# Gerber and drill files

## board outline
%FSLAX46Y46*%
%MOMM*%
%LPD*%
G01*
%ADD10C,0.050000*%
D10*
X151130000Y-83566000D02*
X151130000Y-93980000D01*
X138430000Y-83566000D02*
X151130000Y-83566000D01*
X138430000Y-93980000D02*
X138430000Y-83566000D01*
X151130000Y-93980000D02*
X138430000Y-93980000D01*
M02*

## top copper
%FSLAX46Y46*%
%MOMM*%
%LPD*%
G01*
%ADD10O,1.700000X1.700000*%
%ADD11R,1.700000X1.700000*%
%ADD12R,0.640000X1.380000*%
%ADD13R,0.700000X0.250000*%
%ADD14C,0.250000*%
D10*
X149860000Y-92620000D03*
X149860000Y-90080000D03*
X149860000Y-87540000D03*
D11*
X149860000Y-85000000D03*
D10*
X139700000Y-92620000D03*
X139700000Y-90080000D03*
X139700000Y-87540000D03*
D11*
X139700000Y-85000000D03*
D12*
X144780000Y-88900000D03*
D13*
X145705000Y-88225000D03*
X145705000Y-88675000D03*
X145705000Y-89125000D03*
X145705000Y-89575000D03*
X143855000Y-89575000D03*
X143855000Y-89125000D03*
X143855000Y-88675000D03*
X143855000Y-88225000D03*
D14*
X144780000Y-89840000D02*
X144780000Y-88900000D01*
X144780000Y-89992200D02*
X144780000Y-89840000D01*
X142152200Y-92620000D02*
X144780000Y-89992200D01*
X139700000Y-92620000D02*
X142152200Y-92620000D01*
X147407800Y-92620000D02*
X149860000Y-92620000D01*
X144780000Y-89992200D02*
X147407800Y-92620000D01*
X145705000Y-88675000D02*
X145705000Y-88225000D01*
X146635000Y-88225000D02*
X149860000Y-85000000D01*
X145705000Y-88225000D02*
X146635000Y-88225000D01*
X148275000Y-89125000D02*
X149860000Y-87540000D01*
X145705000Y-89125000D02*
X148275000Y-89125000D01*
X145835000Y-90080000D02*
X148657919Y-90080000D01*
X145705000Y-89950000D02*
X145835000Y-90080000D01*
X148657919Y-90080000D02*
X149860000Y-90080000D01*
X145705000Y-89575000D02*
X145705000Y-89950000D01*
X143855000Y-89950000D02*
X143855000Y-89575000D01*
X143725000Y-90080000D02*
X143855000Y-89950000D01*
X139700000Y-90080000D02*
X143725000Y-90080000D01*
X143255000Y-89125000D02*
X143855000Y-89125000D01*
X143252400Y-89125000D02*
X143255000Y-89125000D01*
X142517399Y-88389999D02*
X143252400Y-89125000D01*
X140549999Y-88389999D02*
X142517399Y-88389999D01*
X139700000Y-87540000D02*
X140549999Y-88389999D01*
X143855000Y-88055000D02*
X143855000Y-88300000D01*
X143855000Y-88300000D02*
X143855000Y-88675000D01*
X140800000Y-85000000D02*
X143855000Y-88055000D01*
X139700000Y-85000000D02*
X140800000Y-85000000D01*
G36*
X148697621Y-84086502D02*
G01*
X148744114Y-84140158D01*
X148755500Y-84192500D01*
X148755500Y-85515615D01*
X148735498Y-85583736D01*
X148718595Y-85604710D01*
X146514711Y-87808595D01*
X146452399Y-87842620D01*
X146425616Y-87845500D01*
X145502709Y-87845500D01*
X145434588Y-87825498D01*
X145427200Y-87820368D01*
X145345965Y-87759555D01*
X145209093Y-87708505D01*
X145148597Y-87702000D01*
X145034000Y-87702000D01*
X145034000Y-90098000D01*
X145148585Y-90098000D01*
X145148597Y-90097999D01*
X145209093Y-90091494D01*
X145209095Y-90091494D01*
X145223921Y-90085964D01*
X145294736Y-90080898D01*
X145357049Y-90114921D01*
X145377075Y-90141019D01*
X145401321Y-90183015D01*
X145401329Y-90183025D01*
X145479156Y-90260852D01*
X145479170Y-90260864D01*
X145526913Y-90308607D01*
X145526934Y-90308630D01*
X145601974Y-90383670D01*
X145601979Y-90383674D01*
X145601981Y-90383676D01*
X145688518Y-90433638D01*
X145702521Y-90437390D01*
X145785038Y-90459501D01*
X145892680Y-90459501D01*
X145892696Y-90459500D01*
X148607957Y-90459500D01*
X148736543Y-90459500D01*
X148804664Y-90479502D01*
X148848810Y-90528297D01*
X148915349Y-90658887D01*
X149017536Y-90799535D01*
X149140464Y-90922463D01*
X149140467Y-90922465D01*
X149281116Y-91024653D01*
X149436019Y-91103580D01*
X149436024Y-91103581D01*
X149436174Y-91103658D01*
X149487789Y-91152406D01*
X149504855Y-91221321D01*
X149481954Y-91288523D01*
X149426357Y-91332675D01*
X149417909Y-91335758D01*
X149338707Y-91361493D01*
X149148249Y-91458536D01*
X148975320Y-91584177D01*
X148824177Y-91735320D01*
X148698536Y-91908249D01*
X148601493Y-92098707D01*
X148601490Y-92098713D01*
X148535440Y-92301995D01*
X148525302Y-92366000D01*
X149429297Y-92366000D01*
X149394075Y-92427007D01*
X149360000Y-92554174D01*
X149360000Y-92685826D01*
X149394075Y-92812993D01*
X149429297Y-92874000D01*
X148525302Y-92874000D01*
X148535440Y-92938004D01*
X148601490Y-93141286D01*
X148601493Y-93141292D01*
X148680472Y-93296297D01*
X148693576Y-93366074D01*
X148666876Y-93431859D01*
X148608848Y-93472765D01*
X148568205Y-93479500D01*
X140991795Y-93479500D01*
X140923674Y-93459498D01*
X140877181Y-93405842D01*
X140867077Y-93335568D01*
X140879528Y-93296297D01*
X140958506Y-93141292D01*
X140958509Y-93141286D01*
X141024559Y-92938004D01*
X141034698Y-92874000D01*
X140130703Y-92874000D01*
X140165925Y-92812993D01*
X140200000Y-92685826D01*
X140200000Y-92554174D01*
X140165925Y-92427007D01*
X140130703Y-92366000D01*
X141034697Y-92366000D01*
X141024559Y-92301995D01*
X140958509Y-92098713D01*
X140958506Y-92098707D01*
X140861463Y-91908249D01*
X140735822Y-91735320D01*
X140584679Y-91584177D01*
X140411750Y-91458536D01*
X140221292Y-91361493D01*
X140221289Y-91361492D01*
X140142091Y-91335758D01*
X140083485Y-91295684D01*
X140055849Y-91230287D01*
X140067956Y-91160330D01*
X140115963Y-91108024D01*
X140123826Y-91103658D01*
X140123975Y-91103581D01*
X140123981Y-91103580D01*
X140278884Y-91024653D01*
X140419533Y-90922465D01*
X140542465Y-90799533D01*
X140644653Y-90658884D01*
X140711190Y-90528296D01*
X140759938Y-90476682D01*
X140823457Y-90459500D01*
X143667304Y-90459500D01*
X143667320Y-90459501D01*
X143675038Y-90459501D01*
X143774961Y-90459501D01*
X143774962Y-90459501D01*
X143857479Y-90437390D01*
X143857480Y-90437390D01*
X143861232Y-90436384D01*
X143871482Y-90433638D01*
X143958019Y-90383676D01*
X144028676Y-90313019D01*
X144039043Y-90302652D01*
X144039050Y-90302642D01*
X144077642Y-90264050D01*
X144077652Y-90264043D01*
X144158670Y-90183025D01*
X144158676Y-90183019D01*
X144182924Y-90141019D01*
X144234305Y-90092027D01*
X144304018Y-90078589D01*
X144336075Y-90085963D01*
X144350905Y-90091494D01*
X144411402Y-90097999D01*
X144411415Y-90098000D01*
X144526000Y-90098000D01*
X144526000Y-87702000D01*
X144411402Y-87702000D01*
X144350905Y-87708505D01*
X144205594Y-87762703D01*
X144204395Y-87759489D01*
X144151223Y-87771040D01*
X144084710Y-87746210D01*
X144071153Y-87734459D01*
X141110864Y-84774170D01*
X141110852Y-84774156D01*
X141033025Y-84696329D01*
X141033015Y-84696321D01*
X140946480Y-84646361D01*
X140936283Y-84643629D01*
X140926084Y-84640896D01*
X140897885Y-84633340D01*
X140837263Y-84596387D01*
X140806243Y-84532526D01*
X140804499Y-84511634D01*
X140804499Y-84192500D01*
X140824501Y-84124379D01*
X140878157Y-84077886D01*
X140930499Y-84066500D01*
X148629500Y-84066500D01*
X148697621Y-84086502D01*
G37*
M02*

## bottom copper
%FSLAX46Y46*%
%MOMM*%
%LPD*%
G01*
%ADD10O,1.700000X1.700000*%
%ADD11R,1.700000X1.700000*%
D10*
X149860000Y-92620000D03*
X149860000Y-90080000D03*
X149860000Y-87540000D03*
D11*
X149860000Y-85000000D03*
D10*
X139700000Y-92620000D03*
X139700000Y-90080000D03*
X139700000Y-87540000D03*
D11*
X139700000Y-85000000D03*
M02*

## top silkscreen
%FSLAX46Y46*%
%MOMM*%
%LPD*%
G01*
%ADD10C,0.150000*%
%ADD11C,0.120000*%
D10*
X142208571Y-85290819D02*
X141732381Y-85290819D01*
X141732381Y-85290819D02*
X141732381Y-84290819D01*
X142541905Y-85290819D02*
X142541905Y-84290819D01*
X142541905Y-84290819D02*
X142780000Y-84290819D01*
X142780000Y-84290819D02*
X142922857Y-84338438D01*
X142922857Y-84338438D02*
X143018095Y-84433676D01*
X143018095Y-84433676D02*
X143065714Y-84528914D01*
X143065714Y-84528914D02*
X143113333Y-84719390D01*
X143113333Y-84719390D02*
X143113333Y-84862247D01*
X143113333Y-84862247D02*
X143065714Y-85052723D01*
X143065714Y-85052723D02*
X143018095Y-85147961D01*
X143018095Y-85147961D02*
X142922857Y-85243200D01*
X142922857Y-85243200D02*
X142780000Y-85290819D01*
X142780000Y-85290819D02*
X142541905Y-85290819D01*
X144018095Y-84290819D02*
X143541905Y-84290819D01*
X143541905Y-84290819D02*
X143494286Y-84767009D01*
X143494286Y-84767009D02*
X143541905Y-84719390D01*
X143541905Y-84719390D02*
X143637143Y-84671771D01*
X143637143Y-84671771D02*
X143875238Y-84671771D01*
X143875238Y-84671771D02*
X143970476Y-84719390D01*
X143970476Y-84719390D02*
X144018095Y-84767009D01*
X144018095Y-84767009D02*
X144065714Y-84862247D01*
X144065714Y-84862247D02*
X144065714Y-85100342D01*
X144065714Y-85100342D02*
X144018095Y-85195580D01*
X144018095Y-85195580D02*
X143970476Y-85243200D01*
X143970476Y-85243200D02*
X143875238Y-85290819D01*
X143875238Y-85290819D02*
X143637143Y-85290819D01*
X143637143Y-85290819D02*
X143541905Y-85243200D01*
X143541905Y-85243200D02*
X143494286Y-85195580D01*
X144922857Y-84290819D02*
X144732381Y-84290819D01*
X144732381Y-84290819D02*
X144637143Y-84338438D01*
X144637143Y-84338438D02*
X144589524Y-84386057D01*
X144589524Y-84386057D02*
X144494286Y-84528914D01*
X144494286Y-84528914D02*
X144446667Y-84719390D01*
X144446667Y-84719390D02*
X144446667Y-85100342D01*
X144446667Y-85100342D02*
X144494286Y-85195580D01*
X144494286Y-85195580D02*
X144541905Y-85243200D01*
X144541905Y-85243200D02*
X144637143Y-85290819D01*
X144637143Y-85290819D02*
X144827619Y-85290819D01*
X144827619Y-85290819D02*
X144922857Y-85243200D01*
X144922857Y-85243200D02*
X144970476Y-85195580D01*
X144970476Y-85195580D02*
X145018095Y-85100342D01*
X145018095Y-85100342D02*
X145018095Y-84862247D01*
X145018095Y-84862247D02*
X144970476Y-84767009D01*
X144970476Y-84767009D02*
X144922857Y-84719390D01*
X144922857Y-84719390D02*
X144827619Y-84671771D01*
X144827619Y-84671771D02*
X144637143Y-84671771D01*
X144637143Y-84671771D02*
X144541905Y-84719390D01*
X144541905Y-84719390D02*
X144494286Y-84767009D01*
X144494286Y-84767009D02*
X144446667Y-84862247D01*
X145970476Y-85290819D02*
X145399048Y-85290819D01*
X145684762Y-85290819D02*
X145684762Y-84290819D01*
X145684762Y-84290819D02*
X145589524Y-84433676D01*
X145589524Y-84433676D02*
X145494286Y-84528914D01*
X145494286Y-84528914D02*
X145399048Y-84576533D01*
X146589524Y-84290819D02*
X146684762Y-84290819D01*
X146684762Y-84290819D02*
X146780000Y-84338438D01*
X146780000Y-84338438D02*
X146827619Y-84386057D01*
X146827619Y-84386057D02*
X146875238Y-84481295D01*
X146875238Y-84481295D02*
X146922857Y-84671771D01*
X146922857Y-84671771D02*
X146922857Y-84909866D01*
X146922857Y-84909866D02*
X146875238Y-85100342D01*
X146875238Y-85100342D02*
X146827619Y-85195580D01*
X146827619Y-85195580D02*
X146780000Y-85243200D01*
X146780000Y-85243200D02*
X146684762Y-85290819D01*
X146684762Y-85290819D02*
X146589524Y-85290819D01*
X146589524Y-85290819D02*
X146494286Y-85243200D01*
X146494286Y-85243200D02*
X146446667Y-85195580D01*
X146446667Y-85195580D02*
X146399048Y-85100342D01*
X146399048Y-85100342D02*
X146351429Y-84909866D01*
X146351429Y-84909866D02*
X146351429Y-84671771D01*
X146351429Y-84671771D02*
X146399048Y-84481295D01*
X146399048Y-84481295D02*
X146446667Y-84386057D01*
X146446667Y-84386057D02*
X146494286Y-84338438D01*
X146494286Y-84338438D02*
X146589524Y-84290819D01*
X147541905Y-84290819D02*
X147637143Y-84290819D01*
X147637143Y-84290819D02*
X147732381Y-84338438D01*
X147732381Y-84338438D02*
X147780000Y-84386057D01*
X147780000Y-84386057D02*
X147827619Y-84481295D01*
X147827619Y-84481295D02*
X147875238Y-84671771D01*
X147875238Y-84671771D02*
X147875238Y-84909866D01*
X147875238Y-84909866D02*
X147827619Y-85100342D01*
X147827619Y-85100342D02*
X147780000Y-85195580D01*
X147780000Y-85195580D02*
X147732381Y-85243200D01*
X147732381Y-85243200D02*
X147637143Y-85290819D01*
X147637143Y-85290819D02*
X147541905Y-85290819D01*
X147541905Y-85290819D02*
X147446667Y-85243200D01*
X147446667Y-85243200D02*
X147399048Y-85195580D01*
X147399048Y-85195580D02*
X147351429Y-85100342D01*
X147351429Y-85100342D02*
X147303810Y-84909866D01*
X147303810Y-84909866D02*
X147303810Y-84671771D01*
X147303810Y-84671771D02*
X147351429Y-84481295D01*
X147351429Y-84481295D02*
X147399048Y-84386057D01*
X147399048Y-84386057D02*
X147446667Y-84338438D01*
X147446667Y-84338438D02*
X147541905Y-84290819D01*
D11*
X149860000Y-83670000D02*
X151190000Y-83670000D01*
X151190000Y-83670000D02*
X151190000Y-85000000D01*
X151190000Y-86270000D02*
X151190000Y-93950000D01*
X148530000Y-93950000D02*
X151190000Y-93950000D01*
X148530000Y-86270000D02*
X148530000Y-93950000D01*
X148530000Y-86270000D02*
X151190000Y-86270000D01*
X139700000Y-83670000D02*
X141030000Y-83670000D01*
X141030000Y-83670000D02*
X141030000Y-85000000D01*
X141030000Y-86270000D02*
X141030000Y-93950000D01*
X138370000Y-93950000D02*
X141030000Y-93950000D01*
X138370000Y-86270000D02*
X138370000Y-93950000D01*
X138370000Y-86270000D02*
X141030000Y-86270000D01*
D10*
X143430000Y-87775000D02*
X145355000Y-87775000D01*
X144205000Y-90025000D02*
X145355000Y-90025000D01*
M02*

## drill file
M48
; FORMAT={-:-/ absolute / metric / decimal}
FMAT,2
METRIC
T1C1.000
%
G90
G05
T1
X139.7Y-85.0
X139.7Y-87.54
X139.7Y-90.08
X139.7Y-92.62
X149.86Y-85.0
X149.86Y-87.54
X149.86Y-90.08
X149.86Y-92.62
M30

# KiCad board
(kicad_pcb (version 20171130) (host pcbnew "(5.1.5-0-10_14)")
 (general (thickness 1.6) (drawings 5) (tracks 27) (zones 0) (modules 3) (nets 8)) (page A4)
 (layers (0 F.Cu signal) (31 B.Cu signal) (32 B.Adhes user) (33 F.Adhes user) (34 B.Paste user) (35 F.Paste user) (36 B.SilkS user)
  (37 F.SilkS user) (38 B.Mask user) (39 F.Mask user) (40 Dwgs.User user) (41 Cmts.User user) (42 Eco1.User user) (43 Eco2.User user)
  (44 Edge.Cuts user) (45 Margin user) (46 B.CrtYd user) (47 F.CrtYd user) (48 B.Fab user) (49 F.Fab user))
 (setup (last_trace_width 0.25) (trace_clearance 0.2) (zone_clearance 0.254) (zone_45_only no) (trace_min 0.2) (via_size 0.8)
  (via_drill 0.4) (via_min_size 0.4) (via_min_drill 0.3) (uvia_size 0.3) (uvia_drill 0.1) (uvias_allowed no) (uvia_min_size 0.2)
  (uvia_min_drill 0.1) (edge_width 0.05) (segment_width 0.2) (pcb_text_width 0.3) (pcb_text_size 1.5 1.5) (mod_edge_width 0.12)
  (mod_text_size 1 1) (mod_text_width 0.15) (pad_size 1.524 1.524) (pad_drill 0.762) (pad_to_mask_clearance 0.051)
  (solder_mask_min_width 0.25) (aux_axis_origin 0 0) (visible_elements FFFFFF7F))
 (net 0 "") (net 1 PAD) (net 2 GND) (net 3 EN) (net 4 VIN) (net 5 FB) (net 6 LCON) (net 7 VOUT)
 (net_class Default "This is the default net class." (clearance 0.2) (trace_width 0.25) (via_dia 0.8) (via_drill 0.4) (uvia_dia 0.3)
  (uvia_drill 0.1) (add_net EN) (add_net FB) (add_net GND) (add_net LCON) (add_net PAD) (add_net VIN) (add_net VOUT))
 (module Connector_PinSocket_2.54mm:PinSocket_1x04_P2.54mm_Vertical (layer F.Cu) (at 149.86 85)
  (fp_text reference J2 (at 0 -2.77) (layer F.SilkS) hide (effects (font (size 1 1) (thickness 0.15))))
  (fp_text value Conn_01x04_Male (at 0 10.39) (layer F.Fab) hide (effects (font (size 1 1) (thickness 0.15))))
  (fp_line (start 0 -1.33) (end 1.33 -1.33) (layer F.SilkS) (width 0.12))
  (fp_line (start 1.33 -1.33) (end 1.33 0) (layer F.SilkS) (width 0.12))
  (fp_line (start 1.33 1.27) (end 1.33 8.95) (layer F.SilkS) (width 0.12))
  (fp_line (start -1.33 8.95) (end 1.33 8.95) (layer F.SilkS) (width 0.12))
  (fp_line (start -1.33 1.27) (end -1.33 8.95) (layer F.SilkS) (width 0.12))
  (fp_line (start -1.33 1.27) (end 1.33 1.27) (layer F.SilkS) (width 0.12))
  (pad 4 thru_hole oval (at 0 7.62) (size 1.7 1.7) (drill 1) (layers *.Cu *.Mask) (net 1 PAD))
  (pad 3 thru_hole oval (at 0 5.08) (size 1.7 1.7) (drill 1) (layers *.Cu *.Mask) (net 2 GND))
  (pad 2 thru_hole oval (at 0 2.54) (size 1.7 1.7) (drill 1) (layers *.Cu *.Mask) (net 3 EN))
  (pad 1 thru_hole rect (at 0 0) (size 1.7 1.7) (drill 1) (layers *.Cu *.Mask) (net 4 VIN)))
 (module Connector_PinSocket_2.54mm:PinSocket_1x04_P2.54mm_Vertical (layer F.Cu) (at 139.7 85)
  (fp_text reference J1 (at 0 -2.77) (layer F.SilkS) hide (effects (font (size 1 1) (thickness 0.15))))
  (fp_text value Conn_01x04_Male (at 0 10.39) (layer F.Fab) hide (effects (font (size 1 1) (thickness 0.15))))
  (fp_line (start 0 -1.33) (end 1.33 -1.33) (layer F.SilkS) (width 0.12))
  (fp_line (start 1.33 -1.33) (end 1.33 0) (layer F.SilkS) (width 0.12))
  (fp_line (start 1.33 1.27) (end 1.33 8.95) (layer F.SilkS) (width 0.12))
  (fp_line (start -1.33 8.95) (end 1.33 8.95) (layer F.SilkS) (width 0.12))
  (fp_line (start -1.33 1.27) (end -1.33 8.95) (layer F.SilkS) (width 0.12))
  (fp_line (start -1.33 1.27) (end 1.33 1.27) (layer F.SilkS) (width 0.12))
  (pad 4 thru_hole oval (at 0 7.62) (size 1.7 1.7) (drill 1) (layers *.Cu *.Mask) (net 1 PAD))
  (pad 3 thru_hole oval (at 0 5.08) (size 1.7 1.7) (drill 1) (layers *.Cu *.Mask) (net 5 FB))
  (pad 2 thru_hole oval (at 0 2.54) (size 1.7 1.7) (drill 1) (layers *.Cu *.Mask) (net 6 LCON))
  (pad 1 thru_hole rect (at 0 0) (size 1.7 1.7) (drill 1) (layers *.Cu *.Mask) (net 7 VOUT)))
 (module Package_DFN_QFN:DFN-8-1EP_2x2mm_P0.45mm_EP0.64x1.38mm (layer F.Cu) (at 144.78 88.9)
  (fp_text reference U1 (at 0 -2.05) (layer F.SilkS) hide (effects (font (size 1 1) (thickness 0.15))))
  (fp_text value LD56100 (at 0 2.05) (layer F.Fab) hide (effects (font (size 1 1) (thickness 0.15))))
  (fp_line (start -1.35 -1.125) (end 0.575 -1.125) (layer F.SilkS) (width 0.15))
  (fp_line (start -0.575 1.125) (end 0.575 1.125) (layer F.SilkS) (width 0.15))
  (pad "" smd rect (at 0 0.345) (size 0.53 0.54) (layers F.Paste))
  (pad "" smd rect (at 0 -0.345) (size 0.53 0.54) (layers F.Paste))
  (pad 9 smd rect (at 0 0) (size 0.64 1.38) (layers F.Cu F.Mask) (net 1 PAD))
  (pad 8 smd rect (at 0.925 -0.675) (size 0.7 0.25) (layers F.Cu F.Paste F.Mask) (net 4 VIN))
  (pad 7 smd rect (at 0.925 -0.225) (size 0.7 0.25) (layers F.Cu F.Paste F.Mask) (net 4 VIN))
  (pad 6 smd rect (at 0.925 0.225) (size 0.7 0.25) (layers F.Cu F.Paste F.Mask) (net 3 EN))
  (pad 5 smd rect (at 0.925 0.675) (size 0.7 0.25) (layers F.Cu F.Paste F.Mask) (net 2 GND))
  (pad 4 smd rect (at -0.925 0.675) (size 0.7 0.25) (layers F.Cu F.Paste F.Mask) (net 5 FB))
  (pad 3 smd rect (at -0.925 0.225) (size 0.7 0.25) (layers F.Cu F.Paste F.Mask) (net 6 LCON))
  (pad 2 smd rect (at -0.925 -0.225) (size 0.7 0.25) (layers F.Cu F.Paste F.Mask) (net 7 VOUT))
  (pad 1 smd rect (at -0.925 -0.675) (size 0.7 0.25) (layers F.Cu F.Paste F.Mask) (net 7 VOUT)))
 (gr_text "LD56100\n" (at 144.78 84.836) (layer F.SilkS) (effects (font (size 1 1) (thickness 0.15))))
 (gr_line (start 151.13 83.566) (end 151.13 93.98) (layer Edge.Cuts) (width 0.05))
 (gr_line (start 138.43 83.566) (end 151.13 83.566) (layer Edge.Cuts) (width 0.05))
 (gr_line (start 138.43 93.98) (end 138.43 83.566) (layer Edge.Cuts) (width 0.05))
 (gr_line (start 151.13 93.98) (end 138.43 93.98) (layer Edge.Cuts) (width 0.05))
 (segment (start 144.78 89.84) (end 144.78 88.9) (width 0.25) (layer F.Cu) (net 1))
 (segment (start 144.78 89.9922) (end 144.78 89.84) (width 0.25) (layer F.Cu) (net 1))
 (segment (start 142.1522 92.62) (end 144.78 89.9922) (width 0.25) (layer F.Cu) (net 1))
 (segment (start 139.7 92.62) (end 142.1522 92.62) (width 0.25) (layer F.Cu) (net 1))
 (segment (start 147.4078 92.62) (end 149.86 92.62) (width 0.25) (layer F.Cu) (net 1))
 (segment (start 144.78 89.9922) (end 147.4078 92.62) (width 0.25) (layer F.Cu) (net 1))
 (segment (start 145.705 88.675) (end 145.705 88.225) (width 0.25) (layer F.Cu) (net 4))
 (segment (start 146.635 88.225) (end 149.86 85) (width 0.25) (layer F.Cu) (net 4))
 (segment (start 145.705 88.225) (end 146.635 88.225) (width 0.25) (layer F.Cu) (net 4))
 (segment (start 148.275 89.125) (end 149.86 87.54) (width 0.25) (layer F.Cu) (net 3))
 (segment (start 145.705 89.125) (end 148.275 89.125) (width 0.25) (layer F.Cu) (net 3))
 (segment (start 145.835 90.08) (end 148.657919 90.08) (width 0.25) (layer F.Cu) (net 2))
 (segment (start 145.705 89.95) (end 145.835 90.08) (width 0.25) (layer F.Cu) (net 2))
 (segment (start 148.657919 90.08) (end 149.86 90.08) (width 0.25) (layer F.Cu) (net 2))
 (segment (start 145.705 89.575) (end 145.705 89.95) (width 0.25) (layer F.Cu) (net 2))
 (segment (start 143.855 89.95) (end 143.855 89.575) (width 0.25) (layer F.Cu) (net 5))
 (segment (start 143.725 90.08) (end 143.855 89.95) (width 0.25) (layer F.Cu) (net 5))
 (segment (start 139.7 90.08) (end 143.725 90.08) (width 0.25) (layer F.Cu) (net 5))
 (segment (start 143.255 89.125) (end 143.855 89.125) (width 0.25) (layer F.Cu) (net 6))
 (segment (start 143.2524 89.125) (end 143.255 89.125) (width 0.25) (layer F.Cu) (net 6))
 (segment (start 142.517399 88.389999) (end 143.2524 89.125) (width 0.25) (layer F.Cu) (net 6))
 (segment (start 140.549999 88.389999) (end 142.517399 88.389999) (width 0.25) (layer F.Cu) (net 6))
 (segment (start 139.7 87.54) (end 140.549999 88.389999) (width 0.25) (layer F.Cu) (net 6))
 (segment (start 143.855 88.055) (end 143.855 88.3) (width 0.25) (layer F.Cu) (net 7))
 (segment (start 143.855 88.3) (end 143.855 88.675) (width 0.25) (layer F.Cu) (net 7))
 (segment (start 140.8 85) (end 143.855 88.055) (width 0.25) (layer F.Cu) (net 7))
 (segment (start 139.7 85) (end 140.8 85) (width 0.25) (layer F.Cu) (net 7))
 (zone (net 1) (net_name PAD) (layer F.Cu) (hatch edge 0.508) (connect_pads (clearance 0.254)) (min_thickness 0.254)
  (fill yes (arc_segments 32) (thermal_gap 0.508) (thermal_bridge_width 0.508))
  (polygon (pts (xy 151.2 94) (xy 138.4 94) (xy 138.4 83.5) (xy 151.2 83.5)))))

